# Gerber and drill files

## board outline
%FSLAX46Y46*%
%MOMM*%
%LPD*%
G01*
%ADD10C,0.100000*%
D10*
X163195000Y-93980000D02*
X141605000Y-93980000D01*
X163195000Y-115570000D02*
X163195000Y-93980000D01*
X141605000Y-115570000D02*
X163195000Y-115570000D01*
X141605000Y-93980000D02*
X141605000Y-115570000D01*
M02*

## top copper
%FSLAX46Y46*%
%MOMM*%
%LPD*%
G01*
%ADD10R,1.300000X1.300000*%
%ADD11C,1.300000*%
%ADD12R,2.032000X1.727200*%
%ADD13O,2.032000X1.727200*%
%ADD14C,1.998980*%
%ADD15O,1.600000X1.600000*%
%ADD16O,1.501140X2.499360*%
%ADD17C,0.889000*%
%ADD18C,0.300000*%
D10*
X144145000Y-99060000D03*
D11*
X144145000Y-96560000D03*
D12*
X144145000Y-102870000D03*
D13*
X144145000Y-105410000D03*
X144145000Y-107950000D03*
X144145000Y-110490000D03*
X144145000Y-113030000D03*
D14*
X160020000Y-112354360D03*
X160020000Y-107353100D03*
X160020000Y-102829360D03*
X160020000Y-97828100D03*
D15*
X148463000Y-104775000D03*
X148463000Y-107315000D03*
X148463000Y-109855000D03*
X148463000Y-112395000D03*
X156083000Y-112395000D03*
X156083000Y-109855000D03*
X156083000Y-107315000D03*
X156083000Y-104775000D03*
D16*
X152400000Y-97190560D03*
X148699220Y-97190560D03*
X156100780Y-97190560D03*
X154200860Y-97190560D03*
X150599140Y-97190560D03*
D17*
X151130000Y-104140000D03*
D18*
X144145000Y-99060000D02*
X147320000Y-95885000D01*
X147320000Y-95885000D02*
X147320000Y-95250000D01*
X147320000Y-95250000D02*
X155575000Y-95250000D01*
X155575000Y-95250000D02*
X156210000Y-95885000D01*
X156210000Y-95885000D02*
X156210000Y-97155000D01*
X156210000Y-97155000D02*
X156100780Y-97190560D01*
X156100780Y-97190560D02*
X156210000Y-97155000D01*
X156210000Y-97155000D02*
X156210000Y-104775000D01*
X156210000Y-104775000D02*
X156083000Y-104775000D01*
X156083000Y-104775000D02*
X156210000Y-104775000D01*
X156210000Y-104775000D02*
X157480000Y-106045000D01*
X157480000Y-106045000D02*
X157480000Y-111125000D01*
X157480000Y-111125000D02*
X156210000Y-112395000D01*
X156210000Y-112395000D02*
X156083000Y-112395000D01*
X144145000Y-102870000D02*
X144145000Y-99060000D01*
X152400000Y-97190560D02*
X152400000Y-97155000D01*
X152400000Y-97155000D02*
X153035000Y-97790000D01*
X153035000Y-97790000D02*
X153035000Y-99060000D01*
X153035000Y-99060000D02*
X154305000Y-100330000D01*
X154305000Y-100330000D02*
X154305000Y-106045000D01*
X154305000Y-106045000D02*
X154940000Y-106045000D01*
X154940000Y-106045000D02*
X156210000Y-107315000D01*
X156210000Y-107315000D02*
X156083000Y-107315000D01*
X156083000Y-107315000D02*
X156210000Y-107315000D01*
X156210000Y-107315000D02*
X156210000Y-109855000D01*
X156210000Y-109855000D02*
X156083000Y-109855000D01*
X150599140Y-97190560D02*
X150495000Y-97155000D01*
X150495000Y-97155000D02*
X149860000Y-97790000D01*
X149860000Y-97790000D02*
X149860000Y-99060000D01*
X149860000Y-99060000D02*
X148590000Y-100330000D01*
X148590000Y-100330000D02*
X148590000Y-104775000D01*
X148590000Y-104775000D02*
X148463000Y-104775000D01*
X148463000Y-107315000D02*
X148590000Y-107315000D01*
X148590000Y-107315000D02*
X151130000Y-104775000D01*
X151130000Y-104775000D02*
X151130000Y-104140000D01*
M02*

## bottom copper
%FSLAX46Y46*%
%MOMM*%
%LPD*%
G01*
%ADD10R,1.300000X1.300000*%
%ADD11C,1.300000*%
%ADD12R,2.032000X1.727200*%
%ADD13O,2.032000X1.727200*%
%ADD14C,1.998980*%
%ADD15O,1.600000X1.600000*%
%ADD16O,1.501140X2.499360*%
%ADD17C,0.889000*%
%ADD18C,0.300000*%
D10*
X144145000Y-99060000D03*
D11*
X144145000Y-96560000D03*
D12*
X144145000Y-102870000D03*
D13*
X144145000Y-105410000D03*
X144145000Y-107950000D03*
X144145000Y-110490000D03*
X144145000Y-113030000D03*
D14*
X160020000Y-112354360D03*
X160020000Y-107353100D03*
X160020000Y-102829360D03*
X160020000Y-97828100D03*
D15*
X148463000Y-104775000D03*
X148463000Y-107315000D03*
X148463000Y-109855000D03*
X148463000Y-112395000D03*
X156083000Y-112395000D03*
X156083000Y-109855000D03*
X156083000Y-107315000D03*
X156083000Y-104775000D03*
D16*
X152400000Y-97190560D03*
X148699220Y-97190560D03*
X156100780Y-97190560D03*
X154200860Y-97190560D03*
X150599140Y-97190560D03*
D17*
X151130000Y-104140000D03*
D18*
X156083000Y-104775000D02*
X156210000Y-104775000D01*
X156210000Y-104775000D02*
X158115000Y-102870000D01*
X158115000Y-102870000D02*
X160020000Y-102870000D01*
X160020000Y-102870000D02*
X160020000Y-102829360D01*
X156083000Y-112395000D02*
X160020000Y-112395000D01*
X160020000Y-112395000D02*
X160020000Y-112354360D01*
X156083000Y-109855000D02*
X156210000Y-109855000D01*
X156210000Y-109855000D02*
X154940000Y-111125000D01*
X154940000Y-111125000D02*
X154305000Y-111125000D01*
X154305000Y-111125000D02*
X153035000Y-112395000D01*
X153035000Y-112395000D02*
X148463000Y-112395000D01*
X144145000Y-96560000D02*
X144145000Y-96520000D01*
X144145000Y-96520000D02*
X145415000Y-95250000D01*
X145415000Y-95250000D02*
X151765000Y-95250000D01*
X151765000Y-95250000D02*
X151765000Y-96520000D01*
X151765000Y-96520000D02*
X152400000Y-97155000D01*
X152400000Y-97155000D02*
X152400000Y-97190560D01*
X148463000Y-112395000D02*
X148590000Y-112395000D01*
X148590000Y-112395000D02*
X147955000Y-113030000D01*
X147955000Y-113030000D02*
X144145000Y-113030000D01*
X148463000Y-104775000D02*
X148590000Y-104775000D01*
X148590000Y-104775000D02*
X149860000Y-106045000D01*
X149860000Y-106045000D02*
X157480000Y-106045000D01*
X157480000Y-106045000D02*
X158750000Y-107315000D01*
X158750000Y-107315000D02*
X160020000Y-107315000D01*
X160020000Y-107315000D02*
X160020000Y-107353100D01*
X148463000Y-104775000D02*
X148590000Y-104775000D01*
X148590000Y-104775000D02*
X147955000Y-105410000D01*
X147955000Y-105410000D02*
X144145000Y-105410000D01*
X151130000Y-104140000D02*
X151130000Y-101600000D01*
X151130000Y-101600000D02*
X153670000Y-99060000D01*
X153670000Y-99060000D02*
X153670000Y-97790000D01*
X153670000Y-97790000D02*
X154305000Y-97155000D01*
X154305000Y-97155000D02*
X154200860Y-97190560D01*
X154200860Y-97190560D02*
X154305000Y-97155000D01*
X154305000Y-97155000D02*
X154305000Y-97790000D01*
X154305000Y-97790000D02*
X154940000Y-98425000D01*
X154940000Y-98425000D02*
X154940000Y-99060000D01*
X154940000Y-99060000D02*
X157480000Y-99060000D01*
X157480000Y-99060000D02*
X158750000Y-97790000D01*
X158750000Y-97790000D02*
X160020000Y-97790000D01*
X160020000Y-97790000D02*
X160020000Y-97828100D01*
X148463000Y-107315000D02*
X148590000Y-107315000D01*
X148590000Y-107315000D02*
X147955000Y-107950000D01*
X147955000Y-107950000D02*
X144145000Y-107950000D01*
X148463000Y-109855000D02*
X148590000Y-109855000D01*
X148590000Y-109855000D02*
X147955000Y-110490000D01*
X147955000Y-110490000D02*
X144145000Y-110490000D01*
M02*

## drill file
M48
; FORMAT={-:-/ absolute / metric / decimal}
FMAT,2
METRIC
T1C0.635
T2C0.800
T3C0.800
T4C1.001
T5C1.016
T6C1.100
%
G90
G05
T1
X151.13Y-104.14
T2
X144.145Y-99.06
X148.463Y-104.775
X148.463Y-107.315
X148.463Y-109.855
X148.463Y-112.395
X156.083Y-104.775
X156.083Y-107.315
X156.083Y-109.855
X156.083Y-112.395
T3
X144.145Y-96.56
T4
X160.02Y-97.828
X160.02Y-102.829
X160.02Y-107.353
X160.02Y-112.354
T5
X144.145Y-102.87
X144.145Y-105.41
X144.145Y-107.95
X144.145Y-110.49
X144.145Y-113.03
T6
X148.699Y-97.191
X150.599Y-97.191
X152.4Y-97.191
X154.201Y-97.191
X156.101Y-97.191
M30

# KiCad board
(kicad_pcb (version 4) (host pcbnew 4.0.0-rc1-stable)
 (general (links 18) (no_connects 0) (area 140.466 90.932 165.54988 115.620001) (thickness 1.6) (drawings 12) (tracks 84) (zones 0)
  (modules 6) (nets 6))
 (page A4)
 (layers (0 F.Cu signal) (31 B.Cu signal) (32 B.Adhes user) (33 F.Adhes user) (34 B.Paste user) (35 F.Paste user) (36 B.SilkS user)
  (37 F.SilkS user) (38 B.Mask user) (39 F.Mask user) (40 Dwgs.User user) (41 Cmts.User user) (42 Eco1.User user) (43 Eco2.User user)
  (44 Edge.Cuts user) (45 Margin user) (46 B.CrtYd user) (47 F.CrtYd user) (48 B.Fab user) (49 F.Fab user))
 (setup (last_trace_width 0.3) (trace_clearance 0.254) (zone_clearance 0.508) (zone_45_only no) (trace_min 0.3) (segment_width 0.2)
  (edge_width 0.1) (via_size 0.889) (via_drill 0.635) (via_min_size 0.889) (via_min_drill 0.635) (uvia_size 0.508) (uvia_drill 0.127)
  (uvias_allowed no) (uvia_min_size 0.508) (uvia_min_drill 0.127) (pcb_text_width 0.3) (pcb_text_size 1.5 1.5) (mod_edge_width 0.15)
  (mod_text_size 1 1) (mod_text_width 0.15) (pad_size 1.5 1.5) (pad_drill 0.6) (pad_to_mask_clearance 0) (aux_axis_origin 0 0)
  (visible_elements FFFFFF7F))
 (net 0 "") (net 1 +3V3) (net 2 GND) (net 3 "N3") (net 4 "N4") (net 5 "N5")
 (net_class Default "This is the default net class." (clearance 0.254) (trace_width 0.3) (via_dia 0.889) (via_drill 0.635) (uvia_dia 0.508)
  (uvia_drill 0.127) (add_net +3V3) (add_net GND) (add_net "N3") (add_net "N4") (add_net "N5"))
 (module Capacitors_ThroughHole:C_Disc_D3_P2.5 (layer F.Cu) (at 144.145 99.06 90)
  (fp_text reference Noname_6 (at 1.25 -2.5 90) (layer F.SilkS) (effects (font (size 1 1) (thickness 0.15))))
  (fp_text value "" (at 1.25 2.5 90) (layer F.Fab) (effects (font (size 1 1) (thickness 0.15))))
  (pad 1 thru_hole rect (at 0 0 90) (size 1.3 1.3) (drill 0.8) (layers *.Cu *.Mask F.SilkS) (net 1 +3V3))
  (pad 2 thru_hole circle (at 2.5 0 90) (size 1.3 1.3) (drill 0.8001) (layers *.Cu *.Mask F.SilkS) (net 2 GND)))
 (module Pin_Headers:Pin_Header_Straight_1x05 (layer F.Cu) (at 144.145 102.87)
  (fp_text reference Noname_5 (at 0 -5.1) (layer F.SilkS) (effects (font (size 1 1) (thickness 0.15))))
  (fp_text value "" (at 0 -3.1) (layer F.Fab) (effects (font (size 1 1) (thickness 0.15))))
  (pad 1 thru_hole rect (at 0 0) (size 2.032 1.7272) (drill 1.016) (layers *.Cu *.Mask F.SilkS) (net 1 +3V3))
  (pad 2 thru_hole oval (at 0 2.54) (size 2.032 1.7272) (drill 1.016) (layers *.Cu *.Mask F.SilkS) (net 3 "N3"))
  (pad 3 thru_hole oval (at 0 5.08) (size 2.032 1.7272) (drill 1.016) (layers *.Cu *.Mask F.SilkS) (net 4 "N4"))
  (pad 4 thru_hole oval (at 0 7.62) (size 2.032 1.7272) (drill 1.016) (layers *.Cu *.Mask F.SilkS) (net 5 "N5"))
  (pad 5 thru_hole oval (at 0 10.16) (size 2.032 1.7272) (drill 1.016) (layers *.Cu *.Mask F.SilkS) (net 2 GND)))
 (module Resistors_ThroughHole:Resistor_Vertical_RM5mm (layer F.Cu) (at 160.02 109.855 90)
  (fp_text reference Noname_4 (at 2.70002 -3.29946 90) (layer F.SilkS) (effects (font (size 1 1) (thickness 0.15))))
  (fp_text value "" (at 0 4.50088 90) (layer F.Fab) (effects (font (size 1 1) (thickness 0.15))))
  (pad 1 thru_hole circle (at -2.49936 0 90) (size 1.99898 1.99898) (drill 1.00076) (layers *.Cu *.SilkS *.Mask) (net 1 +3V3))
  (pad 2 thru_hole circle (at 2.5019 0 90) (size 1.99898 1.99898) (drill 1.00076) (layers *.Cu *.SilkS *.Mask) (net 3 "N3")))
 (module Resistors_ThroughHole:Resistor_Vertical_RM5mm (layer F.Cu) (at 160.02 100.33 90)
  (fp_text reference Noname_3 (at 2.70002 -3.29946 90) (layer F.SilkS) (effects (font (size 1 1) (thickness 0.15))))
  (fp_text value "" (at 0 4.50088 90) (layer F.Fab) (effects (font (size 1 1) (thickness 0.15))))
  (pad 1 thru_hole circle (at -2.49936 0 90) (size 1.99898 1.99898) (drill 1.00076) (layers *.Cu *.SilkS *.Mask) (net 1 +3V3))
  (pad 2 thru_hole circle (at 2.5019 0 90) (size 1.99898 1.99898) (drill 1.00076) (layers *.Cu *.SilkS *.Mask) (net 4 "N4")))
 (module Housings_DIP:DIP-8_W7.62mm (layer F.Cu) (at 148.463 104.775)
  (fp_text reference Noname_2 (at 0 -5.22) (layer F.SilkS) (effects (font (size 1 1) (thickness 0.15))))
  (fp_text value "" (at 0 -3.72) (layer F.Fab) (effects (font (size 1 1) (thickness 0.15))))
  (pad 1 thru_hole oval (at 0 0) (size 1.6 1.6) (drill 0.8) (layers *.Cu *.Mask F.SilkS) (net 3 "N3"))
  (pad 2 thru_hole oval (at 0 2.54) (size 1.6 1.6) (drill 0.8) (layers *.Cu *.Mask F.SilkS) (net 4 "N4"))
  (pad 3 thru_hole oval (at 0 5.08) (size 1.6 1.6) (drill 0.8) (layers *.Cu *.Mask F.SilkS) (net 5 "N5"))
  (pad 4 thru_hole oval (at 0 7.62) (size 1.6 1.6) (drill 0.8) (layers *.Cu *.Mask F.SilkS) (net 2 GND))
  (pad 5 thru_hole oval (at 7.62 7.62) (size 1.6 1.6) (drill 0.8) (layers *.Cu *.Mask F.SilkS) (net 1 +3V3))
  (pad 6 thru_hole oval (at 7.62 5.08) (size 1.6 1.6) (drill 0.8) (layers *.Cu *.Mask F.SilkS) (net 2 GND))
  (pad 7 thru_hole oval (at 7.62 2.54) (size 1.6 1.6) (drill 0.8) (layers *.Cu *.Mask F.SilkS) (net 2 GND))
  (pad 8 thru_hole oval (at 7.62 0) (size 1.6 1.6) (drill 0.8) (layers *.Cu *.Mask F.SilkS) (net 1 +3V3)))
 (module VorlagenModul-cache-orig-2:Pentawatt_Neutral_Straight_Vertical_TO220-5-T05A (layer F.Cu) (at 152.4 97.79)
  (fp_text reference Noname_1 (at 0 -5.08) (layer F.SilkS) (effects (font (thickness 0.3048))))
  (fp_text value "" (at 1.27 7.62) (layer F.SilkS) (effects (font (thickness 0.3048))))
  (pad 3 thru_hole oval (at 0 -0.59944 90) (size 2.49936 1.50114) (drill 1.09982) (layers *.Cu *.Mask F.SilkS) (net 2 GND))
  (pad 1 thru_hole oval (at -3.70078 -0.59944 90) (size 2.49936 1.50114) (drill 1.09982) (layers *.Cu *.Mask F.SilkS))
  (pad 5 thru_hole oval (at 3.70078 -0.59944 90) (size 2.49936 1.50114) (drill 1.09982) (layers *.Cu *.Mask F.SilkS) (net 1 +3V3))
  (pad 4 thru_hole oval (at 1.80086 -0.59944 90) (size 2.49936 1.50114) (drill 1.09982) (layers *.Cu *.Mask F.SilkS) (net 4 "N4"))
  (pad 2 thru_hole oval (at -1.80086 -0.59944 90) (size 2.49936 1.50114) (drill 1.09982) (layers *.Cu *.Mask F.SilkS) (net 3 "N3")))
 (gr_line (start 163.195 93.98) (end 141.605 93.98) (angle 90) (layer Edge.Cuts) (width 0.1))
 (gr_line (start 163.195 115.57) (end 163.195 93.98) (angle 90) (layer Edge.Cuts) (width 0.1))
 (gr_line (start 141.605 115.57) (end 163.195 115.57) (angle 90) (layer Edge.Cuts) (width 0.1))
 (gr_line (start 141.605 93.98) (end 141.605 115.57) (angle 90) (layer Edge.Cuts) (width 0.1))
 (segment (start 144.145 99.06) (end 147.32 95.885) (width 0.3) (layer F.Cu) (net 1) (status 80000))
 (segment (start 147.32 95.885) (end 147.32 95.25) (width 0.3) (layer F.Cu) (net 1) (status 80000))
 (segment (start 147.32 95.25) (end 155.575 95.25) (width 0.3) (layer F.Cu) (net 1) (status 80000))
 (segment (start 155.575 95.25) (end 156.21 95.885) (width 0.3) (layer F.Cu) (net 1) (status 80000))
 (segment (start 156.21 95.885) (end 156.21 97.155) (width 0.3) (layer F.Cu) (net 1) (status 80000))
 (segment (start 156.21 97.155) (end 156.10078 97.19056) (width 0.3) (layer F.Cu) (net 1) (status 80000))
 (segment (start 156.083 104.775) (end 156.21 104.775) (width 0.3) (layer B.Cu) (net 1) (status 80000))
 (segment (start 156.21 104.775) (end 158.115 102.87) (width 0.3) (layer B.Cu) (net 1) (status 80000))
 (segment (start 158.115 102.87) (end 160.02 102.87) (width 0.3) (layer B.Cu) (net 1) (status 80000))
 (segment (start 160.02 102.87) (end 160.02 102.82936) (width 0.3) (layer B.Cu) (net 1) (status 80000))
 (segment (start 156.10078 97.19056) (end 156.21 97.155) (width 0.3) (layer F.Cu) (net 1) (status 80000))
 (segment (start 156.21 97.155) (end 156.21 104.775) (width 0.3) (layer F.Cu) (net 1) (status 80000))
 (segment (start 156.21 104.775) (end 156.083 104.775) (width 0.3) (layer F.Cu) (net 1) (status 80000))
 (segment (start 156.083 104.775) (end 156.21 104.775) (width 0.3) (layer F.Cu) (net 1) (status 80000))
 (segment (start 156.21 104.775) (end 157.48 106.045) (width 0.3) (layer F.Cu) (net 1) (status 80000))
 (segment (start 157.48 106.045) (end 157.48 111.125) (width 0.3) (layer F.Cu) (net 1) (status 80000))
 (segment (start 157.48 111.125) (end 156.21 112.395) (width 0.3) (layer F.Cu) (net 1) (status 80000))
 (segment (start 156.21 112.395) (end 156.083 112.395) (width 0.3) (layer F.Cu) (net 1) (status 80000))
 (segment (start 156.083 112.395) (end 160.02 112.395) (width 0.3) (layer B.Cu) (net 1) (status 80000))
 (segment (start 160.02 112.395) (end 160.02 112.35436) (width 0.3) (layer B.Cu) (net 1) (status 80000))
 (segment (start 144.145 102.87) (end 144.145 99.06) (width 0.3) (layer F.Cu) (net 1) (status 80000))
 (segment (start 152.4 97.19056) (end 152.4 97.155) (width 0.3) (layer F.Cu) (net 2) (status 80000))
 (segment (start 152.4 97.155) (end 153.035 97.79) (width 0.3) (layer F.Cu) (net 2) (status 80000))
 (segment (start 153.035 97.79) (end 153.035 99.06) (width 0.3) (layer F.Cu) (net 2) (status 80000))
 (segment (start 153.035 99.06) (end 154.305 100.33) (width 0.3) (layer F.Cu) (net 2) (status 80000))
 (segment (start 154.305 100.33) (end 154.305 106.045) (width 0.3) (layer F.Cu) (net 2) (status 80000))
 (segment (start 154.305 106.045) (end 154.94 106.045) (width 0.3) (layer F.Cu) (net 2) (status 80000))
 (segment (start 154.94 106.045) (end 156.21 107.315) (width 0.3) (layer F.Cu) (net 2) (status 80000))
 (segment (start 156.21 107.315) (end 156.083 107.315) (width 0.3) (layer F.Cu) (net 2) (status 80000))
 (segment (start 156.083 109.855) (end 156.21 109.855) (width 0.3) (layer B.Cu) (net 2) (status 80000))
 (segment (start 156.21 109.855) (end 154.94 111.125) (width 0.3) (layer B.Cu) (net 2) (status 80000))
 (segment (start 154.94 111.125) (end 154.305 111.125) (width 0.3) (layer B.Cu) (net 2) (status 80000))
 (segment (start 154.305 111.125) (end 153.035 112.395) (width 0.3) (layer B.Cu) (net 2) (status 80000))
 (segment (start 153.035 112.395) (end 148.463 112.395) (width 0.3) (layer B.Cu) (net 2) (status 80000))
 (segment (start 144.145 96.56) (end 144.145 96.52) (width 0.3) (layer B.Cu) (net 2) (status 80000))
 (segment (start 144.145 96.52) (end 145.415 95.25) (width 0.3) (layer B.Cu) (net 2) (status 80000))
 (segment (start 145.415 95.25) (end 151.765 95.25) (width 0.3) (layer B.Cu) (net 2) (status 80000))
 (segment (start 151.765 95.25) (end 151.765 96.52) (width 0.3) (layer B.Cu) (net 2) (status 80000))
 (segment (start 151.765 96.52) (end 152.4 97.155) (width 0.3) (layer B.Cu) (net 2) (status 80000))
 (segment (start 152.4 97.155) (end 152.4 97.19056) (width 0.3) (layer B.Cu) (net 2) (status 80000))
 (segment (start 148.463 112.395) (end 148.59 112.395) (width 0.3) (layer B.Cu) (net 2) (status 80000))
 (segment (start 148.59 112.395) (end 147.955 113.03) (width 0.3) (layer B.Cu) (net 2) (status 80000))
 (segment (start 147.955 113.03) (end 144.145 113.03) (width 0.3) (layer B.Cu) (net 2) (status 80000))
 (segment (start 156.083 107.315) (end 156.21 107.315) (width 0.3) (layer F.Cu) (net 2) (status 80000))
 (segment (start 156.21 107.315) (end 156.21 109.855) (width 0.3) (layer F.Cu) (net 2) (status 80000))
 (segment (start 156.21 109.855) (end 156.083 109.855) (width 0.3) (layer F.Cu) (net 2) (status 80000))
 (segment (start 148.463 104.775) (end 148.59 104.775) (width 0.3) (layer B.Cu) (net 3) (status 80000))
 (segment (start 148.59 104.775) (end 149.86 106.045) (width 0.3) (layer B.Cu) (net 3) (status 80000))
 (segment (start 149.86 106.045) (end 157.48 106.045) (width 0.3) (layer B.Cu) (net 3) (status 80000))
 (segment (start 157.48 106.045) (end 158.75 107.315) (width 0.3) (layer B.Cu) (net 3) (status 80000))
 (segment (start 158.75 107.315) (end 160.02 107.315) (width 0.3) (layer B.Cu) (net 3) (status 80000))
 (segment (start 160.02 107.315) (end 160.02 107.3531) (width 0.3) (layer B.Cu) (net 3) (status 80000))
 (segment (start 150.59914 97.19056) (end 150.495 97.155) (width 0.3) (layer F.Cu) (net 3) (status 80000))
 (segment (start 150.495 97.155) (end 149.86 97.79) (width 0.3) (layer F.Cu) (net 3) (status 80000))
 (segment (start 149.86 97.79) (end 149.86 99.06) (width 0.3) (layer F.Cu) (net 3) (status 80000))
 (segment (start 149.86 99.06) (end 148.59 100.33) (width 0.3) (layer F.Cu) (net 3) (status 80000))
 (segment (start 148.59 100.33) (end 148.59 104.775) (width 0.3) (layer F.Cu) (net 3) (status 80000))
 (segment (start 148.59 104.775) (end 148.463 104.775) (width 0.3) (layer F.Cu) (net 3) (status 80000))
 (segment (start 148.463 104.775) (end 148.59 104.775) (width 0.3) (layer B.Cu) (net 3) (status 80000))
 (segment (start 148.59 104.775) (end 147.955 105.41) (width 0.3) (layer B.Cu) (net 3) (status 80000))
 (segment (start 147.955 105.41) (end 144.145 105.41) (width 0.3) (layer B.Cu) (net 3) (status 80000))
 (segment (start 148.463 107.315) (end 148.59 107.315) (width 0.3) (layer F.Cu) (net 4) (status 80000))
 (segment (start 148.59 107.315) (end 151.13 104.775) (width 0.3) (layer F.Cu) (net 4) (status 80000))
 (segment (start 151.13 104.775) (end 151.13 104.14) (width 0.3) (layer F.Cu) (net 4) (status 80000))
 (segment (start 151.13 104.14) (end 151.13 101.6) (width 0.3) (layer B.Cu) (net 4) (status 80000))
 (segment (start 151.13 101.6) (end 153.67 99.06) (width 0.3) (layer B.Cu) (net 4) (status 80000))
 (segment (start 153.67 99.06) (end 153.67 97.79) (width 0.3) (layer B.Cu) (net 4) (status 80000))
 (segment (start 153.67 97.79) (end 154.305 97.155) (width 0.3) (layer B.Cu) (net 4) (status 80000))
 (segment (start 154.305 97.155) (end 154.20086 97.19056) (width 0.3) (layer B.Cu) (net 4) (status 80000))
 (segment (start 154.20086 97.19056) (end 154.305 97.155) (width 0.3) (layer B.Cu) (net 4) (status 80000))
 (segment (start 154.305 97.155) (end 154.305 97.79) (width 0.3) (layer B.Cu) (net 4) (status 80000))
 (segment (start 154.305 97.79) (end 154.94 98.425) (width 0.3) (layer B.Cu) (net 4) (status 80000))
 (segment (start 154.94 98.425) (end 154.94 99.06) (width 0.3) (layer B.Cu) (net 4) (status 80000))
 (segment (start 154.94 99.06) (end 157.48 99.06) (width 0.3) (layer B.Cu) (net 4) (status 80000))
 (segment (start 157.48 99.06) (end 158.75 97.79) (width 0.3) (layer B.Cu) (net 4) (status 80000))
 (segment (start 158.75 97.79) (end 160.02 97.79) (width 0.3) (layer B.Cu) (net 4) (status 80000))
 (segment (start 160.02 97.79) (end 160.02 97.8281) (width 0.3) (layer B.Cu) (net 4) (status 80000))
 (segment (start 148.463 107.315) (end 148.59 107.315) (width 0.3) (layer B.Cu) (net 4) (status 80000))
 (segment (start 148.59 107.315) (end 147.955 107.95) (width 0.3) (layer B.Cu) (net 4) (status 80000))
 (segment (start 147.955 107.95) (end 144.145 107.95) (width 0.3) (layer B.Cu) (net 4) (status 80000))
 (segment (start 148.463 109.855) (end 148.59 109.855) (width 0.3) (layer B.Cu) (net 5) (status 80000))
 (segment (start 148.59 109.855) (end 147.955 110.49) (width 0.3) (layer B.Cu) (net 5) (status 80000))
 (segment (start 147.955 110.49) (end 144.145 110.49) (width 0.3) (layer B.Cu) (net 5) (status 80000))
 (via (at 151.13 104.14) (size 0.889) (layers F.Cu B.Cu) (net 4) (status 80000)))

